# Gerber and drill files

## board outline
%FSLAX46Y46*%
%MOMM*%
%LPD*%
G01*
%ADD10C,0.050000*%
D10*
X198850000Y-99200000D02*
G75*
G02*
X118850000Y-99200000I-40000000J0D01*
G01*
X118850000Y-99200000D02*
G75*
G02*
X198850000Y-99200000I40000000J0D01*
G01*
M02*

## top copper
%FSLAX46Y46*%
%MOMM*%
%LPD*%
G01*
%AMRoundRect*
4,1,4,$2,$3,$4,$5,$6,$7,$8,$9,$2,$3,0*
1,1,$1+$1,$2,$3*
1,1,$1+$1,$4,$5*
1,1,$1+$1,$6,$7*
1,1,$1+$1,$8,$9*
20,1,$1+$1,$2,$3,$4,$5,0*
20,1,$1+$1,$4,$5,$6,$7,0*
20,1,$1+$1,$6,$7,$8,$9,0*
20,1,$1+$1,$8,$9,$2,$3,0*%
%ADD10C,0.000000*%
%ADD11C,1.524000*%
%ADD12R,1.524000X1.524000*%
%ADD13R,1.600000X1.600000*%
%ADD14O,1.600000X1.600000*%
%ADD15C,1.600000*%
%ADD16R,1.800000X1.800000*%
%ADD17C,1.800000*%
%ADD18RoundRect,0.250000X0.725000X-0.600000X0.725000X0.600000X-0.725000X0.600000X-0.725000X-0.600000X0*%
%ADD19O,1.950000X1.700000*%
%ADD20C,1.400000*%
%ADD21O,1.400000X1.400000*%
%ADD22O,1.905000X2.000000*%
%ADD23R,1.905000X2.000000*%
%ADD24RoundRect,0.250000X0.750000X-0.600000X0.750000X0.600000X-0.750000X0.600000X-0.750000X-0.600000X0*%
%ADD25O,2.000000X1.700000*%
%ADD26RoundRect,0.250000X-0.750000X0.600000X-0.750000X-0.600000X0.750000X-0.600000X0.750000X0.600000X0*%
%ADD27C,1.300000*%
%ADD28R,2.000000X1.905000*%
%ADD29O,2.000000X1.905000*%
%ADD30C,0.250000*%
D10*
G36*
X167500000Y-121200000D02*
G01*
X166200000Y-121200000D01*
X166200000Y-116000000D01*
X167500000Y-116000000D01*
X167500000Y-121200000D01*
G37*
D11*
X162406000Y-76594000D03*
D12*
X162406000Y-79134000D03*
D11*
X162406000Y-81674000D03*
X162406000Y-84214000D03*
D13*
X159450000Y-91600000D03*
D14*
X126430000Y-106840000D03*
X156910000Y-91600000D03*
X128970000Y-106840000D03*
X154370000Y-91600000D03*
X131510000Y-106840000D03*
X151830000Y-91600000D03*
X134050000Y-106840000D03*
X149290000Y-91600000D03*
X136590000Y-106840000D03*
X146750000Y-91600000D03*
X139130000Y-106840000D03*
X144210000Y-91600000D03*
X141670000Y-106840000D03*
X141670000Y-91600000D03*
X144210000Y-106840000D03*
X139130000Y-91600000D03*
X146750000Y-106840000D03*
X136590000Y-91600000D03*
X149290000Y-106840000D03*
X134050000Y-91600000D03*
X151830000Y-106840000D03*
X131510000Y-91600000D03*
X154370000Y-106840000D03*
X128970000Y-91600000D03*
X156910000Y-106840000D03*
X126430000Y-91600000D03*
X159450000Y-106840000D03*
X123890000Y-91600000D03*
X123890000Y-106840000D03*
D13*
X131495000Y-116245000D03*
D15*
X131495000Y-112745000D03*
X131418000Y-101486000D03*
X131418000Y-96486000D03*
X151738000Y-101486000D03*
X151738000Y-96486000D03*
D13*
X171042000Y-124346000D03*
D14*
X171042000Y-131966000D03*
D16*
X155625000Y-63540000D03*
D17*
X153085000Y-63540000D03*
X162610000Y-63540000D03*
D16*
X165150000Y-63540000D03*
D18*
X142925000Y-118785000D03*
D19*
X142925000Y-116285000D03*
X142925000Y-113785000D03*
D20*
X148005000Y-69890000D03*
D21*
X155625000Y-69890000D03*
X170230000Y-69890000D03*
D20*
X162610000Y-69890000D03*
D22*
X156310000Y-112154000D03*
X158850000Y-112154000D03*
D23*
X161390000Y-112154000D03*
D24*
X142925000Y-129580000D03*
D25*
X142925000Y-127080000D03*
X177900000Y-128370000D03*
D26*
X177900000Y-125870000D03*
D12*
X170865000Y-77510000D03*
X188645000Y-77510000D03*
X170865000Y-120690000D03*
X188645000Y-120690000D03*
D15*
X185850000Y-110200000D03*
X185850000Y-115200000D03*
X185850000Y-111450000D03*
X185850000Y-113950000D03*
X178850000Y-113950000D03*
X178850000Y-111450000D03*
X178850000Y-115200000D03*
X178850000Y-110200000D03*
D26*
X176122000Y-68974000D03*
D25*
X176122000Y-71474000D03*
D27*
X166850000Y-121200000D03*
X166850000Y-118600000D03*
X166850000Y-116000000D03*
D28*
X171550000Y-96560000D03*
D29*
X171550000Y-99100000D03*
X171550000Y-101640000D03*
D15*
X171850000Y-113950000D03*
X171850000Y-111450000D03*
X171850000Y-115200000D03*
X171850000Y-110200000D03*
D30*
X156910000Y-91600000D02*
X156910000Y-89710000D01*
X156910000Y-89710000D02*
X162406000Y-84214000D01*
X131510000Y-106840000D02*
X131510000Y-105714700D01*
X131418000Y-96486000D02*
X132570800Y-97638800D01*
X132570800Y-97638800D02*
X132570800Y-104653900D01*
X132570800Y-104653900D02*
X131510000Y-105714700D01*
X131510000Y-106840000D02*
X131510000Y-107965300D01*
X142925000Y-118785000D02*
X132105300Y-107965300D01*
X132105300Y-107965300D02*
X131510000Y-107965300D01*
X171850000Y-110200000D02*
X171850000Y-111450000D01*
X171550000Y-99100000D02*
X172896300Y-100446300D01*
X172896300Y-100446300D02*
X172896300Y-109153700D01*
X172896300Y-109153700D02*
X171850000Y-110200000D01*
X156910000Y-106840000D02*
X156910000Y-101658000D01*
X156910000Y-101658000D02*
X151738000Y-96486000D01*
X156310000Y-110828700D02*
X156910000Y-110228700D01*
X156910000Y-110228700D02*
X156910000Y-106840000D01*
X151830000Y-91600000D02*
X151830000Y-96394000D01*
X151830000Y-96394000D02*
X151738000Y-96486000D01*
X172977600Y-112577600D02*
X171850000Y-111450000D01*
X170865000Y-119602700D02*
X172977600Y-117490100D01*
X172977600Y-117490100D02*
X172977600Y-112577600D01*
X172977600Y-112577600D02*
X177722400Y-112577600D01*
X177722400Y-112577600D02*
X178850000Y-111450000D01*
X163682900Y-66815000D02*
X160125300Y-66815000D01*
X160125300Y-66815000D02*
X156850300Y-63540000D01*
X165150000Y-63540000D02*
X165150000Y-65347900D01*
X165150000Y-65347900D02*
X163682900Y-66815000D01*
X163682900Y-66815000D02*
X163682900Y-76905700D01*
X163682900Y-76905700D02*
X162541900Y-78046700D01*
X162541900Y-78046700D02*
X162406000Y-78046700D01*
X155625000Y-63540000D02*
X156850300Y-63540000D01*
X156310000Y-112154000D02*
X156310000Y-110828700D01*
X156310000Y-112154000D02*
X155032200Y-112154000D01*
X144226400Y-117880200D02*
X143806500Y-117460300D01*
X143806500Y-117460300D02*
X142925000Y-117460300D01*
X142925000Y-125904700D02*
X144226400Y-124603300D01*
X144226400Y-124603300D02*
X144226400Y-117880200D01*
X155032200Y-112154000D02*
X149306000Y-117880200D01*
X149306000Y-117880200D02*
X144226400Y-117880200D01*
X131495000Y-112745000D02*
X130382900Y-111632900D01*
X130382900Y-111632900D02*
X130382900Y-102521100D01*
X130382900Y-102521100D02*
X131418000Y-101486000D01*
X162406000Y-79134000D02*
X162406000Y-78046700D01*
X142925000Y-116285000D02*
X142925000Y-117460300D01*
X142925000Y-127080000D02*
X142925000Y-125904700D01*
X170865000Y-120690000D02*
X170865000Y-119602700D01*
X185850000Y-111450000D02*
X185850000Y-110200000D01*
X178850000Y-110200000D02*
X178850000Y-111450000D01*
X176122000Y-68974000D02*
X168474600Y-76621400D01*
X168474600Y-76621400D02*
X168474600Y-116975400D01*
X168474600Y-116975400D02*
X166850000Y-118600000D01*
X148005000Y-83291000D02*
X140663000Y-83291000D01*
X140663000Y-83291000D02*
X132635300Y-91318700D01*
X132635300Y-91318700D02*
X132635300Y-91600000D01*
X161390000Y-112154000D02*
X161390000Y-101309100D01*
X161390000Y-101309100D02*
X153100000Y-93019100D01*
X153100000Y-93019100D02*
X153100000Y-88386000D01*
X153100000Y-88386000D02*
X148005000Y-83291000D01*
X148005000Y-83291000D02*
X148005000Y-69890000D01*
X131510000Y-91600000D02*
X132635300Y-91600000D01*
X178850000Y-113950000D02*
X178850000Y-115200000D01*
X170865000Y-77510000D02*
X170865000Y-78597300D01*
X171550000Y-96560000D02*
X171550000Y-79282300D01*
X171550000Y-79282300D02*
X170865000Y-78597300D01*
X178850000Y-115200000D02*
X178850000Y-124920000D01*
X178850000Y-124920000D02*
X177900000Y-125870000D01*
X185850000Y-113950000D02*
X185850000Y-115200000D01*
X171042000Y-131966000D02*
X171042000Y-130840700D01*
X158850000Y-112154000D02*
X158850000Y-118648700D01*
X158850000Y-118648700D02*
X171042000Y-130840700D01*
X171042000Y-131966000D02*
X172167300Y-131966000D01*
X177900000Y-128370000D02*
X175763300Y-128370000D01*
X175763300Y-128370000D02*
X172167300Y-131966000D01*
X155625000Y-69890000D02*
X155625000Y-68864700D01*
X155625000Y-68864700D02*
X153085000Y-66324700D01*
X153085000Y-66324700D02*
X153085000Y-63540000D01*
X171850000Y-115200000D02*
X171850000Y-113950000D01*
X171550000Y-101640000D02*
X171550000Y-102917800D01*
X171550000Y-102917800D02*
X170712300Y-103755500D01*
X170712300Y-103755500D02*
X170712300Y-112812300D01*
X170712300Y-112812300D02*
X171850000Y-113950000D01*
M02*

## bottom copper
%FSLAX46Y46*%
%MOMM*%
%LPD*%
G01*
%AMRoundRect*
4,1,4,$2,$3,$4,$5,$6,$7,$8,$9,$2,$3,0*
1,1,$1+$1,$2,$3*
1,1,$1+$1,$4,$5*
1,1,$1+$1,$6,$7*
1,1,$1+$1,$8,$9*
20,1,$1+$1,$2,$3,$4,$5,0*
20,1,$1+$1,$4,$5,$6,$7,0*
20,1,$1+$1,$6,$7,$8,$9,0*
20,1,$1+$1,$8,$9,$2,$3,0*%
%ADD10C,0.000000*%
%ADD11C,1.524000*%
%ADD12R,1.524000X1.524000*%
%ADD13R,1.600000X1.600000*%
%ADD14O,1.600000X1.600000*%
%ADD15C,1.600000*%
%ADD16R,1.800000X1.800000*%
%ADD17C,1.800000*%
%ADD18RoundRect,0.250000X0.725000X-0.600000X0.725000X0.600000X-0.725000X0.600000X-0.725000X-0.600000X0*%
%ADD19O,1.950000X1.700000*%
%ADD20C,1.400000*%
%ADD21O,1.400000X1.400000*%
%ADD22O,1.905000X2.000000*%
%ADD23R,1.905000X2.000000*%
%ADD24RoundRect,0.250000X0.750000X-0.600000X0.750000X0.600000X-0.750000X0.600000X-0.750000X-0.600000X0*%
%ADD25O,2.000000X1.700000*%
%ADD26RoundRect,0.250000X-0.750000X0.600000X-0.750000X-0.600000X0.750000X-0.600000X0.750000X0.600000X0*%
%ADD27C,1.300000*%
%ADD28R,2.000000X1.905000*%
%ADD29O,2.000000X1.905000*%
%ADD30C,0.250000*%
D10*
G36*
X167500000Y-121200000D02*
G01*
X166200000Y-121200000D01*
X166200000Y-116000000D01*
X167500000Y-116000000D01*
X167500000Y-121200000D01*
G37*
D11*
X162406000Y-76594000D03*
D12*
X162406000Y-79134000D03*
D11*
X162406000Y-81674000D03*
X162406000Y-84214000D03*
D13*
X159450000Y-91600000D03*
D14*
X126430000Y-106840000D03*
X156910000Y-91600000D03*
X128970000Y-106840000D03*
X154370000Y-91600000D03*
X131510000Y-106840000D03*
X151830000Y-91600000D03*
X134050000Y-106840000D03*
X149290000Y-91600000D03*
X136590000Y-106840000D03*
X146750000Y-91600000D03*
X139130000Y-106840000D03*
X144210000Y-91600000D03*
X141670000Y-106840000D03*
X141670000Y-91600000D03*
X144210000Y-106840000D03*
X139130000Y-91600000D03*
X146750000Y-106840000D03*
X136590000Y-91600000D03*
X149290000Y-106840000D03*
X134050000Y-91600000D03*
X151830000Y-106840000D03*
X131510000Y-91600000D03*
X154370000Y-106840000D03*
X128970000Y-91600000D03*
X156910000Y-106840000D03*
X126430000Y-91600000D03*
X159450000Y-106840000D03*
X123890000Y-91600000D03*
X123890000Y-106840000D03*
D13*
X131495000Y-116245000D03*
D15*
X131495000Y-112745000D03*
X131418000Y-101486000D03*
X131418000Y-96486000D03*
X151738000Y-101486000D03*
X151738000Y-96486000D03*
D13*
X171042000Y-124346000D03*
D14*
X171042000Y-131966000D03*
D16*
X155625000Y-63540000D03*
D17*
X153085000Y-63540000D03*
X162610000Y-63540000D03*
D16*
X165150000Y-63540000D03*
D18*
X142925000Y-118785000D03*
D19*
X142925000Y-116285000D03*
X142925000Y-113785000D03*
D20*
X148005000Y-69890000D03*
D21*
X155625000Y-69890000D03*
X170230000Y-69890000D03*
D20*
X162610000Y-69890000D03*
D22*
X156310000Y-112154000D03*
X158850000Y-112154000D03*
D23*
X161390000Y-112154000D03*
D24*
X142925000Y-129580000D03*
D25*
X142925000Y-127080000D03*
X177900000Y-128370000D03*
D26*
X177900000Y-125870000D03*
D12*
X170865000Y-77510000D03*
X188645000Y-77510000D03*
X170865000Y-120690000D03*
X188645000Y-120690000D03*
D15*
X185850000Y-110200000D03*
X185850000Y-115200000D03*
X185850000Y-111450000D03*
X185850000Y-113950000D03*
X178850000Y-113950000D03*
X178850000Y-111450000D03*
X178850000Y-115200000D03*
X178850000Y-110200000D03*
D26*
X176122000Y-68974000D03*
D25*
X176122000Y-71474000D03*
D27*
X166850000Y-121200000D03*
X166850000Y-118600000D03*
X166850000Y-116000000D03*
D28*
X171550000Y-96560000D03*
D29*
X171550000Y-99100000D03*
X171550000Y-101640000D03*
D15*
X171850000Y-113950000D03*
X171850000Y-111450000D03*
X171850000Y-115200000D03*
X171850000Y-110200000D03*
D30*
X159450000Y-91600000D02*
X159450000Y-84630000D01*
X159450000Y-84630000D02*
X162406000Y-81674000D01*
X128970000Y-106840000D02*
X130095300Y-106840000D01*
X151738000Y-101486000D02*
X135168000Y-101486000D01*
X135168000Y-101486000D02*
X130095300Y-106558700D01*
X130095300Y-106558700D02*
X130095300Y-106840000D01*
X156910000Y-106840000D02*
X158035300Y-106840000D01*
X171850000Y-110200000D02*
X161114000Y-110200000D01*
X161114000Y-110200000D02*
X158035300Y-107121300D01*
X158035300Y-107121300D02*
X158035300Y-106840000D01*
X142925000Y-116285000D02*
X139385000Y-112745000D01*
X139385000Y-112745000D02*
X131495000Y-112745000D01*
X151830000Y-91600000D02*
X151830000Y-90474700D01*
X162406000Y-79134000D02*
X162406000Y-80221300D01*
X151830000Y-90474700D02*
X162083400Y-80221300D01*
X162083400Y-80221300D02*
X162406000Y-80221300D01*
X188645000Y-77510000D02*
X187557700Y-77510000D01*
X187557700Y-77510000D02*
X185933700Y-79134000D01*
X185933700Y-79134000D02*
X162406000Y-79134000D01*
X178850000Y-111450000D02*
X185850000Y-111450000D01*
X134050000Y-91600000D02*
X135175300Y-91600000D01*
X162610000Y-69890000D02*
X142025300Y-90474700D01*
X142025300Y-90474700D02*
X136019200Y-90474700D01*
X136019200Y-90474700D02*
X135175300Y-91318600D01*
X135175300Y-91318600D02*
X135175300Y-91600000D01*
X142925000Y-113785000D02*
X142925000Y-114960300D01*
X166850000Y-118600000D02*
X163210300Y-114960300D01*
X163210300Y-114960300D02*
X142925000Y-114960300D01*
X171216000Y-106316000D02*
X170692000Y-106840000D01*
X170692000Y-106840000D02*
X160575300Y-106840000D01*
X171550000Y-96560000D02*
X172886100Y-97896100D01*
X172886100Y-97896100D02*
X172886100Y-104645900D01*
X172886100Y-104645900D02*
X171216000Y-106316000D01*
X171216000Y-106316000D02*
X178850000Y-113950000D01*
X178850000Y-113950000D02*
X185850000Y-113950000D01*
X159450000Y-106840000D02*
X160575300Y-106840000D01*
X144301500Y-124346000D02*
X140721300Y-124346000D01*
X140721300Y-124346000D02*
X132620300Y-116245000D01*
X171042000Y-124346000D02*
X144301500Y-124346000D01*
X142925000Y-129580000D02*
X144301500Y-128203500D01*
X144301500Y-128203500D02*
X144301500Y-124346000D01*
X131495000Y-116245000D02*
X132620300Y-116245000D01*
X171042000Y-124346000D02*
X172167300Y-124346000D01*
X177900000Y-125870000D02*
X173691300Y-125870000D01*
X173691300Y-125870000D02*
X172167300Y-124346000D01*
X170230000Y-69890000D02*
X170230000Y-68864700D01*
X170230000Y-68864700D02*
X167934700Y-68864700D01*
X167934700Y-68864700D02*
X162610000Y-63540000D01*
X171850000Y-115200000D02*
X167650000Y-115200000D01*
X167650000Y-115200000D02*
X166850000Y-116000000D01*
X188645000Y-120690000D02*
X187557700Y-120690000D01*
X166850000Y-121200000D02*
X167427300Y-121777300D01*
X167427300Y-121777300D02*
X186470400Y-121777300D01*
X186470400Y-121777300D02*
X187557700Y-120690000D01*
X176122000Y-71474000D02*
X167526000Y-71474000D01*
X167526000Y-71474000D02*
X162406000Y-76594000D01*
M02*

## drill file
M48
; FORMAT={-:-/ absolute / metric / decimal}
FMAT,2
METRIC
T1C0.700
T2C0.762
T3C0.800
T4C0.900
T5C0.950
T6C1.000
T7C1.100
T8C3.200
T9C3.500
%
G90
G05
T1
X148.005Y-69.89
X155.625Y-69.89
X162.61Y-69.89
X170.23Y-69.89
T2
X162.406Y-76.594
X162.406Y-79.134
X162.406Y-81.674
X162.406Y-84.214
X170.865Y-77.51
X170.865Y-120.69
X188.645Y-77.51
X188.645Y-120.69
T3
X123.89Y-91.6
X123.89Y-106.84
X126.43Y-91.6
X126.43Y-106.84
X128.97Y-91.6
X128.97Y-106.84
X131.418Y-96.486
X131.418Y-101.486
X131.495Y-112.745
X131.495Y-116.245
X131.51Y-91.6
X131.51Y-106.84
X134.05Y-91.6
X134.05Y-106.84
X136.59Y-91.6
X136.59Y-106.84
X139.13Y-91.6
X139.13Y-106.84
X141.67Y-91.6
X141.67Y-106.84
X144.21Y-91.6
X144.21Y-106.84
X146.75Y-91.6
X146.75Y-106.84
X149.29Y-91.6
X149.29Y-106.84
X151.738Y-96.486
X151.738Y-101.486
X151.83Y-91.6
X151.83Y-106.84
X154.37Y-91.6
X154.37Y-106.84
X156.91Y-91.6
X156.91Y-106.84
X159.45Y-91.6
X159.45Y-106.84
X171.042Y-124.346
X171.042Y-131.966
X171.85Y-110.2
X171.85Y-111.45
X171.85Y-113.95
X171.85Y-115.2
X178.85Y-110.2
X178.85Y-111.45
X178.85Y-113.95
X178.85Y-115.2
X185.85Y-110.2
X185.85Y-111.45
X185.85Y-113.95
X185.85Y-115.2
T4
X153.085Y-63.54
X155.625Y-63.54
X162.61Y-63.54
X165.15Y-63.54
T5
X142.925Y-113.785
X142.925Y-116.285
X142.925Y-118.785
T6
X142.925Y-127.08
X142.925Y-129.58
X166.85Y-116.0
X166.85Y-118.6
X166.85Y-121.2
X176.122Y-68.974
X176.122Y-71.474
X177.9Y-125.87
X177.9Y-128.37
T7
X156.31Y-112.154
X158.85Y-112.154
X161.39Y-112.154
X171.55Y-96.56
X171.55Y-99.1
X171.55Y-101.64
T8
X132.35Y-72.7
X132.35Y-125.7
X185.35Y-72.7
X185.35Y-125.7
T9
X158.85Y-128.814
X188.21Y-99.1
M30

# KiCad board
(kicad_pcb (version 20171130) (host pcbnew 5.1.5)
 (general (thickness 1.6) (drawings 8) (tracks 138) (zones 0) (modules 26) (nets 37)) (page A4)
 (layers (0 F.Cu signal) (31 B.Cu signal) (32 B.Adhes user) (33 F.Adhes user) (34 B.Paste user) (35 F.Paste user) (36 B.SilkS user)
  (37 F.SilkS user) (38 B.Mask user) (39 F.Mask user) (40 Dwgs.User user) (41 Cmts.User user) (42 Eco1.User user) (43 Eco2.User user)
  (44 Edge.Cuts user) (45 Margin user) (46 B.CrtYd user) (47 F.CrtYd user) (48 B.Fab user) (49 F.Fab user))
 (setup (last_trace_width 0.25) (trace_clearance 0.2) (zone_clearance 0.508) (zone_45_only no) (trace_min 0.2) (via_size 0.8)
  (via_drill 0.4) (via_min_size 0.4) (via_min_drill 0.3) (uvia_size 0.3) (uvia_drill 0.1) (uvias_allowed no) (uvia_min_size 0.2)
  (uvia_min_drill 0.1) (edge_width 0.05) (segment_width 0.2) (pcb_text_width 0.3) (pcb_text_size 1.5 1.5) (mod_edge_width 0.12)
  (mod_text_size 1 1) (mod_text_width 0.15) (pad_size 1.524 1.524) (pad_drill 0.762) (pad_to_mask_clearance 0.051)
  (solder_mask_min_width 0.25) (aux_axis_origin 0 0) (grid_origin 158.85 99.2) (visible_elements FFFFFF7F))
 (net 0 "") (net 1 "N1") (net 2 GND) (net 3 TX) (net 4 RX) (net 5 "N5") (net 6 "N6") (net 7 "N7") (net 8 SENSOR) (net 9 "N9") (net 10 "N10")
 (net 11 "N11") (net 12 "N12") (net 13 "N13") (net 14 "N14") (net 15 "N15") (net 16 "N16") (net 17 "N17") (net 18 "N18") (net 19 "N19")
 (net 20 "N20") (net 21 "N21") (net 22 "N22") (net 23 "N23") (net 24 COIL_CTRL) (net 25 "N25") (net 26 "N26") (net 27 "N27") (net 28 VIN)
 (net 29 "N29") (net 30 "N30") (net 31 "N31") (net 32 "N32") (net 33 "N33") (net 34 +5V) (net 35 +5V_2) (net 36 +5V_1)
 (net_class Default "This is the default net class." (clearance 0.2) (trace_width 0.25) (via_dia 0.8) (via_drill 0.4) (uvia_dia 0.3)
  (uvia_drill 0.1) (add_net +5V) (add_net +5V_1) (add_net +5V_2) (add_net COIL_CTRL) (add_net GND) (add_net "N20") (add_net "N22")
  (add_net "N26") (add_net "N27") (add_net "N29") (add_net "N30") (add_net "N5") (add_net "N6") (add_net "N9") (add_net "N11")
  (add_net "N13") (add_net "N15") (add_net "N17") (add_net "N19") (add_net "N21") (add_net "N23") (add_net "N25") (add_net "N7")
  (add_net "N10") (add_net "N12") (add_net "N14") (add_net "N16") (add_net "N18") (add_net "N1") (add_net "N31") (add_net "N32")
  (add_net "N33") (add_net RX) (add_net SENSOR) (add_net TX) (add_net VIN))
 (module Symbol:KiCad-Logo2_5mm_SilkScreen (layer F.Cu) (at 158.85 135.2)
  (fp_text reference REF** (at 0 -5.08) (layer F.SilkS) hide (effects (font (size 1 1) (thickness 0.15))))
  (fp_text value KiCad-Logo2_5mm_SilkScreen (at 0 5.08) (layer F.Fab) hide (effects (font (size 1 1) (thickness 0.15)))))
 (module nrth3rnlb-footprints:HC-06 (layer F.Cu) (at 166.216 72.784 270)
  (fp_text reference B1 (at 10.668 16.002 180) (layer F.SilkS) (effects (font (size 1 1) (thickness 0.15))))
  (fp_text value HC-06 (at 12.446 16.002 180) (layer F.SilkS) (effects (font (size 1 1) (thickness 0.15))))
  (pad 1 thru_hole circle (at 3.81 3.81 270) (size 1.524 1.524) (drill 0.762) (layers *.Cu *.Mask) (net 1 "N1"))
  (pad 2 thru_hole rect (at 6.35 3.81 270) (size 1.524 1.524) (drill 0.762) (layers *.Cu *.Mask) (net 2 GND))
  (pad 3 thru_hole circle (at 8.89 3.81 270) (size 1.524 1.524) (drill 0.762) (layers *.Cu *.Mask) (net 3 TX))
  (pad 4 thru_hole circle (at 11.43 3.81 270) (size 1.524 1.524) (drill 0.762) (layers *.Cu *.Mask) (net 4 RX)))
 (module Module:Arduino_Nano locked (layer F.Cu) (at 159.45 91.6 270)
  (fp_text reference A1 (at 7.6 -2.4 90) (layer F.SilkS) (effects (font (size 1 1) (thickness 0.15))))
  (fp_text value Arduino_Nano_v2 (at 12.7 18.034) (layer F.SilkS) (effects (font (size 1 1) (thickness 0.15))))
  (pad 1 thru_hole rect (at 0 0 270) (size 1.6 1.6) (drill 0.8) (layers *.Cu *.Mask) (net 3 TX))
  (pad 17 thru_hole oval (at 15.24 33.02 270) (size 1.6 1.6) (drill 0.8) (layers *.Cu *.Mask) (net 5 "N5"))
  (pad 2 thru_hole oval (at 0 2.54 270) (size 1.6 1.6) (drill 0.8) (layers *.Cu *.Mask) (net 4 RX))
  (pad 18 thru_hole oval (at 15.24 30.48 270) (size 1.6 1.6) (drill 0.8) (layers *.Cu *.Mask) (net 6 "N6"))
  (pad 3 thru_hole oval (at 0 5.08 270) (size 1.6 1.6) (drill 0.8) (layers *.Cu *.Mask) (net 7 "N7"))
  (pad 19 thru_hole oval (at 15.24 27.94 270) (size 1.6 1.6) (drill 0.8) (layers *.Cu *.Mask) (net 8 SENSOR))
  (pad 4 thru_hole oval (at 0 7.62 270) (size 1.6 1.6) (drill 0.8) (layers *.Cu *.Mask) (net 2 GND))
  (pad 20 thru_hole oval (at 15.24 25.4 270) (size 1.6 1.6) (drill 0.8) (layers *.Cu *.Mask) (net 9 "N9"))
  (pad 5 thru_hole oval (at 0 10.16 270) (size 1.6 1.6) (drill 0.8) (layers *.Cu *.Mask) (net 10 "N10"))
  (pad 21 thru_hole oval (at 15.24 22.86 270) (size 1.6 1.6) (drill 0.8) (layers *.Cu *.Mask) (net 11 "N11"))
  (pad 6 thru_hole oval (at 0 12.7 270) (size 1.6 1.6) (drill 0.8) (layers *.Cu *.Mask) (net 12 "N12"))
  (pad 22 thru_hole oval (at 15.24 20.32 270) (size 1.6 1.6) (drill 0.8) (layers *.Cu *.Mask) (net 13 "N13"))
  (pad 7 thru_hole oval (at 0 15.24 270) (size 1.6 1.6) (drill 0.8) (layers *.Cu *.Mask) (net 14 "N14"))
  (pad 23 thru_hole oval (at 15.24 17.78 270) (size 1.6 1.6) (drill 0.8) (layers *.Cu *.Mask) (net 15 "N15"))
  (pad 8 thru_hole oval (at 0 17.78 270) (size 1.6 1.6) (drill 0.8) (layers *.Cu *.Mask) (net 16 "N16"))
  (pad 24 thru_hole oval (at 15.24 15.24 270) (size 1.6 1.6) (drill 0.8) (layers *.Cu *.Mask) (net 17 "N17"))
  (pad 9 thru_hole oval (at 0 20.32 270) (size 1.6 1.6) (drill 0.8) (layers *.Cu *.Mask) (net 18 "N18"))
  (pad 25 thru_hole oval (at 15.24 12.7 270) (size 1.6 1.6) (drill 0.8) (layers *.Cu *.Mask) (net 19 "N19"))
  (pad 10 thru_hole oval (at 0 22.86 270) (size 1.6 1.6) (drill 0.8) (layers *.Cu *.Mask) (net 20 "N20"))
  (pad 26 thru_hole oval (at 15.24 10.16 270) (size 1.6 1.6) (drill 0.8) (layers *.Cu *.Mask) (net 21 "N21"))
  (pad 11 thru_hole oval (at 0 25.4 270) (size 1.6 1.6) (drill 0.8) (layers *.Cu *.Mask) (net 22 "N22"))
  (pad 27 thru_hole oval (at 15.24 7.62 270) (size 1.6 1.6) (drill 0.8) (layers *.Cu *.Mask) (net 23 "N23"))
  (pad 12 thru_hole oval (at 0 27.94 270) (size 1.6 1.6) (drill 0.8) (layers *.Cu *.Mask) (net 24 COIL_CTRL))
  (pad 28 thru_hole oval (at 15.24 5.08 270) (size 1.6 1.6) (drill 0.8) (layers *.Cu *.Mask) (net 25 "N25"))
  (pad 13 thru_hole oval (at 0 30.48 270) (size 1.6 1.6) (drill 0.8) (layers *.Cu *.Mask) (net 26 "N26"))
  (pad 29 thru_hole oval (at 15.24 2.54 270) (size 1.6 1.6) (drill 0.8) (layers *.Cu *.Mask) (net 2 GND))
  (pad 14 thru_hole oval (at 0 33.02 270) (size 1.6 1.6) (drill 0.8) (layers *.Cu *.Mask) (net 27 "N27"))
  (pad 30 thru_hole oval (at 15.24 0 270) (size 1.6 1.6) (drill 0.8) (layers *.Cu *.Mask) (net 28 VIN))
  (pad 15 thru_hole oval (at 0 35.56 270) (size 1.6 1.6) (drill 0.8) (layers *.Cu *.Mask) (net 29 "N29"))
  (pad 16 thru_hole oval (at 15.24 35.56 270) (size 1.6 1.6) (drill 0.8) (layers *.Cu *.Mask) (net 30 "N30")))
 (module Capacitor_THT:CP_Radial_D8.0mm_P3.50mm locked (layer F.Cu) (at 131.495 116.245 90)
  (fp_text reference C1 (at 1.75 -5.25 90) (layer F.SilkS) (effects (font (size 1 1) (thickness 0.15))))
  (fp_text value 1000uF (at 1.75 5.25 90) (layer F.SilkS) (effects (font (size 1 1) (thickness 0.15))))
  (pad 1 thru_hole rect (at 0 0 90) (size 1.6 1.6) (drill 0.8) (layers *.Cu *.Mask) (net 28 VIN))
  (pad 2 thru_hole circle (at 3.5 0 90) (size 1.6 1.6) (drill 0.8) (layers *.Cu *.Mask) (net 2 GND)))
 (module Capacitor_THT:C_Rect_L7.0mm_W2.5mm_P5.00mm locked (layer F.Cu) (at 131.418 96.486 270)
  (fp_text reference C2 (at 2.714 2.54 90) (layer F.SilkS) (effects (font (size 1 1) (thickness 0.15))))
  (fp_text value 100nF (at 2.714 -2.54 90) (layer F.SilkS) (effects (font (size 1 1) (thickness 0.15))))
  (pad 2 thru_hole circle (at 5 0 270) (size 1.6 1.6) (drill 0.8) (layers *.Cu *.Mask) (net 2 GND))
  (pad 1 thru_hole circle (at 0 0 270) (size 1.6 1.6) (drill 0.8) (layers *.Cu *.Mask) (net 8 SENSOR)))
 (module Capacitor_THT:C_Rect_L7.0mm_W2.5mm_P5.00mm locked (layer F.Cu) (at 151.738 101.486 90)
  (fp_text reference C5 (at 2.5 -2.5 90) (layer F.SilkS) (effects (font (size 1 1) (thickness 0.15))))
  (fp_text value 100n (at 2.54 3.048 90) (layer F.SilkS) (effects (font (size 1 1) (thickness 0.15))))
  (pad 1 thru_hole circle (at 0 0 90) (size 1.6 1.6) (drill 0.8) (layers *.Cu *.Mask) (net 6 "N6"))
  (pad 2 thru_hole circle (at 5 0 90) (size 1.6 1.6) (drill 0.8) (layers *.Cu *.Mask) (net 2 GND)))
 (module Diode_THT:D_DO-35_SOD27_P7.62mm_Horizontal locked (layer F.Cu) (at 171.042 124.346 270)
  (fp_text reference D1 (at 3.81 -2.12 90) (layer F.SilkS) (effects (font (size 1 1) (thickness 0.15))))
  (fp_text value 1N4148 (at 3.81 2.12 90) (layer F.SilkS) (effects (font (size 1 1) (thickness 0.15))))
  (pad 1 thru_hole rect (at 0 0 270) (size 1.6 1.6) (drill 0.8) (layers *.Cu *.Mask) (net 28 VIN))
  (pad 2 thru_hole oval (at 7.62 0 270) (size 1.6 1.6) (drill 0.8) (layers *.Cu *.Mask) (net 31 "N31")))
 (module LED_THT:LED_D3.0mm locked (layer F.Cu) (at 155.625 63.54 180)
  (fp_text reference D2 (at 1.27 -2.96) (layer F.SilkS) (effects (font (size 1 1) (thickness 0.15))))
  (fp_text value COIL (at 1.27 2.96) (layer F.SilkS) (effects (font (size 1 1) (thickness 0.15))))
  (pad 1 thru_hole rect (at 0 0 180) (size 1.8 1.8) (drill 0.9) (layers *.Cu *.Mask) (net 2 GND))
  (pad 2 thru_hole circle (at 2.54 0 180) (size 1.8 1.8) (drill 0.9) (layers *.Cu *.Mask) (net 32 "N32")))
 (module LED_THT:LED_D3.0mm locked (layer F.Cu) (at 165.15 63.54 180)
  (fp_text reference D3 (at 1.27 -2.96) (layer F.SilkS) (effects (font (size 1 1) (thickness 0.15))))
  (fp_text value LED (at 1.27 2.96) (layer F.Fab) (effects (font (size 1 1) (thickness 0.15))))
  (pad 2 thru_hole circle (at 2.54 0 180) (size 1.8 1.8) (drill 0.9) (layers *.Cu *.Mask) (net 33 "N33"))
  (pad 1 thru_hole rect (at 0 0 180) (size 1.8 1.8) (drill 0.9) (layers *.Cu *.Mask) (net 2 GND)))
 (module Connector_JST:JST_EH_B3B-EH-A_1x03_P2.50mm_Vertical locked (layer F.Cu) (at 142.925 118.785 90)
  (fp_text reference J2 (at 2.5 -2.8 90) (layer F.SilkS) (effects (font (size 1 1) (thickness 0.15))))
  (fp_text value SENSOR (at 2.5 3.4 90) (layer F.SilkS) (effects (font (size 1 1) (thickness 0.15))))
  (pad 1 thru_hole roundrect (at 0 0 90) (size 1.7 1.95) (drill 0.95) (layers *.Cu *.Mask) (roundrect_rratio 0.147059) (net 8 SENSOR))
  (pad 2 thru_hole oval (at 2.5 0 90) (size 1.7 1.95) (drill 0.95) (layers *.Cu *.Mask) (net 2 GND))
  (pad 3 thru_hole oval (at 5 0 90) (size 1.7 1.95) (drill 0.95) (layers *.Cu *.Mask) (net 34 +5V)))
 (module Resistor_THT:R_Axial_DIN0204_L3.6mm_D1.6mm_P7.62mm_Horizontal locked (layer F.Cu) (at 148.005 69.89)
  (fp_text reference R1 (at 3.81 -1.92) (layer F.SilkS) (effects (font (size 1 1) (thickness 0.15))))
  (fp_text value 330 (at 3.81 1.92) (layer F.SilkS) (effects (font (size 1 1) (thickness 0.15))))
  (pad 1 thru_hole circle (at 0 0) (size 1.4 1.4) (drill 0.7) (layers *.Cu *.Mask) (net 24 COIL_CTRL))
  (pad 2 thru_hole oval (at 7.62 0) (size 1.4 1.4) (drill 0.7) (layers *.Cu *.Mask) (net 32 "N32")))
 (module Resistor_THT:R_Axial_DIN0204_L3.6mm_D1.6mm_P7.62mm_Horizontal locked (layer F.Cu) (at 162.61 69.89)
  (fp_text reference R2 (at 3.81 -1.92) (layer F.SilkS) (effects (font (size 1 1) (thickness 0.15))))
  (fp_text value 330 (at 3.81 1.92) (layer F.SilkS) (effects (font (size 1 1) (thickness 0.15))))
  (pad 2 thru_hole oval (at 7.62 0) (size 1.4 1.4) (drill 0.7) (layers *.Cu *.Mask) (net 33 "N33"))
  (pad 1 thru_hole circle (at 0 0) (size 1.4 1.4) (drill 0.7) (layers *.Cu *.Mask) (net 22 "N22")))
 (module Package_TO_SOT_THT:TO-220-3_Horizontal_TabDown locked (layer F.Cu) (at 161.39 112.154 180)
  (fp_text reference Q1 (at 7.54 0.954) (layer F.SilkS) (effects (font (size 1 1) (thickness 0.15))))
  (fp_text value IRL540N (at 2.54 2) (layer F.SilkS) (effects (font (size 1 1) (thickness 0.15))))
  (pad 3 thru_hole oval (at 5.08 0 180) (size 1.905 2) (drill 1.1) (layers *.Cu *.Mask) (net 2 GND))
  (pad 2 thru_hole oval (at 2.54 0 180) (size 1.905 2) (drill 1.1) (layers *.Cu *.Mask) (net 31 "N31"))
  (pad 1 thru_hole rect (at 0 0 180) (size 1.905 2) (drill 1.1) (layers *.Cu *.Mask) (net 24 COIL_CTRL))
  (pad "" np_thru_hole oval (at 2.54 -16.66 180) (size 3.5 3.5) (drill 3.5) (layers *.Cu *.Mask)))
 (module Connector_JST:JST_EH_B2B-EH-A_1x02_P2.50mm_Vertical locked (layer F.Cu) (at 142.925 129.58 90)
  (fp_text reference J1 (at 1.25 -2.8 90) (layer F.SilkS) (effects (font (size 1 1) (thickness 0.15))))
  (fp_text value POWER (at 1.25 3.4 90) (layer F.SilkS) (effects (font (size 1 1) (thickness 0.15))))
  (pad 1 thru_hole roundrect (at 0 0 90) (size 1.7 2) (drill 1) (layers *.Cu *.Mask) (roundrect_rratio 0.147059) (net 28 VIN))
  (pad 2 thru_hole oval (at 2.5 0 90) (size 1.7 2) (drill 1) (layers *.Cu *.Mask) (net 2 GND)))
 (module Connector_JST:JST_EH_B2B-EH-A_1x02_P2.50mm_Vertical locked (layer F.Cu) (at 177.9 125.87 270)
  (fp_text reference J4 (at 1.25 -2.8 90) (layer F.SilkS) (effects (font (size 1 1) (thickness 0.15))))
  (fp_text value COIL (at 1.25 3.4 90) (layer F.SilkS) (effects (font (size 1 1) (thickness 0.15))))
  (pad 2 thru_hole oval (at 2.5 0 270) (size 1.7 2) (drill 1) (layers *.Cu *.Mask) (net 31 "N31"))
  (pad 1 thru_hole roundrect (at 0 0 270) (size 1.7 2) (drill 1) (layers *.Cu *.Mask) (roundrect_rratio 0.147059) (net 28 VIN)))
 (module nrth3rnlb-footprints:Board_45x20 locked (layer F.Cu) (at 179.755 72.43)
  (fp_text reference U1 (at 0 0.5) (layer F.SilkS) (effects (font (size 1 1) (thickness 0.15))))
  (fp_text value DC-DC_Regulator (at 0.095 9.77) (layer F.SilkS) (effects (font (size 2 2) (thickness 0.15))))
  (pad 1 thru_hole rect (at -8.89 5.08) (size 1.524 1.524) (drill 0.762) (layers *.Cu *.Mask) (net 28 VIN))
  (pad 4 thru_hole rect (at 8.89 5.08) (size 1.524 1.524) (drill 0.762) (layers *.Cu *.Mask) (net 2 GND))
  (pad 2 thru_hole rect (at -8.89 48.26) (size 1.524 1.524) (drill 0.762) (layers *.Cu *.Mask) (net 2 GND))
  (pad 3 thru_hole rect (at 8.89 48.26) (size 1.524 1.524) (drill 0.762) (layers *.Cu *.Mask) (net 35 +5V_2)))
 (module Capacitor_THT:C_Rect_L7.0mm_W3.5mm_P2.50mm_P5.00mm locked (layer F.Cu) (at 185.85 115.2 90)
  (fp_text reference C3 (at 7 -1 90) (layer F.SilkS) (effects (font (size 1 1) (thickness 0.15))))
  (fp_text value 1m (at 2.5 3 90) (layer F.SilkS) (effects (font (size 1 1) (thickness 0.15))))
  (pad 2 thru_hole circle (at 5 0 90) (size 1.6 1.6) (drill 0.8) (layers *.Cu *.Mask) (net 2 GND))
  (pad 1 thru_hole circle (at 0 0 90) (size 1.6 1.6) (drill 0.8) (layers *.Cu *.Mask) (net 28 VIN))
  (pad 2 thru_hole circle (at 3.75 0 90) (size 1.6 1.6) (drill 0.8) (layers *.Cu *.Mask) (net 2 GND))
  (pad 1 thru_hole circle (at 1.25 0 90) (size 1.6 1.6) (drill 0.8) (layers *.Cu *.Mask) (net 28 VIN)))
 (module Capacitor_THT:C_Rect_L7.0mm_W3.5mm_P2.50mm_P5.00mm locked (layer F.Cu) (at 178.85 115.2 90)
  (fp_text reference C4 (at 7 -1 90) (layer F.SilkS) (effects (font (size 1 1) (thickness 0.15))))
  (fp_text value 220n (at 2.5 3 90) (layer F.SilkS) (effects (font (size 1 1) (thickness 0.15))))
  (pad 1 thru_hole circle (at 1.25 0 90) (size 1.6 1.6) (drill 0.8) (layers *.Cu *.Mask) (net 28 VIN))
  (pad 2 thru_hole circle (at 3.75 0 90) (size 1.6 1.6) (drill 0.8) (layers *.Cu *.Mask) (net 2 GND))
  (pad 1 thru_hole circle (at 0 0 90) (size 1.6 1.6) (drill 0.8) (layers *.Cu *.Mask) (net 28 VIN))
  (pad 2 thru_hole circle (at 5 0 90) (size 1.6 1.6) (drill 0.8) (layers *.Cu *.Mask) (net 2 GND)))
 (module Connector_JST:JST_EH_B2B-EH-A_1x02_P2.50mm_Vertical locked (layer F.Cu) (at 176.122 68.974 270)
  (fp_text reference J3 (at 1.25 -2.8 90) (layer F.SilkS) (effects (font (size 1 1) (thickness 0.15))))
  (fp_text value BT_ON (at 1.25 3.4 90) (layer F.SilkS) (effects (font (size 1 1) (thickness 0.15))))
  (pad 1 thru_hole roundrect (at 0 0 270) (size 1.7 2) (drill 1) (layers *.Cu *.Mask) (roundrect_rratio 0.147059) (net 34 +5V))
  (pad 2 thru_hole oval (at 2.5 0 270) (size 1.7 2) (drill 1) (layers *.Cu *.Mask) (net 1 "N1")))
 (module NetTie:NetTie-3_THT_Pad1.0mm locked (layer F.Cu) (at 166.85 121.2 90)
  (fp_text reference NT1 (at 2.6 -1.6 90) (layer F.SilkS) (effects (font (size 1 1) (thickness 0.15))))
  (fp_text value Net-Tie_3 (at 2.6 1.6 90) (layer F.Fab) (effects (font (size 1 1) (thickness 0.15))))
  (fp_poly (pts (xy 0 -0.65) (xy 5.2 -0.65) (xy 5.2 0.65) (xy 0 0.65)) (layer F.Cu) (width 0))
  (fp_poly (pts (xy 0 -0.65) (xy 5.2 -0.65) (xy 5.2 0.65) (xy 0 0.65)) (layer B.Cu) (width 0))
  (pad 1 thru_hole circle (at 0 0 90) (size 1.3 1.3) (drill 1) (layers *.Cu) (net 35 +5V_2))
  (pad 2 thru_hole circle (at 2.6 0 90) (size 1.3 1.3) (drill 1) (layers *.Cu) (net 34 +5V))
  (pad 3 thru_hole circle (at 5.2 0 90) (size 1.3 1.3) (drill 1) (layers *.Cu) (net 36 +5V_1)))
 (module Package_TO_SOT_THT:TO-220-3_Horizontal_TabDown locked (layer F.Cu) (at 171.55 96.56 270)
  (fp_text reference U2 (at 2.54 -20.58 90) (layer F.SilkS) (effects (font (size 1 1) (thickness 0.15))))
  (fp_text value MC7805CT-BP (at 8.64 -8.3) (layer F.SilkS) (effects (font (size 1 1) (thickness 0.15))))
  (pad "" np_thru_hole oval (at 2.54 -16.66 270) (size 3.5 3.5) (drill 3.5) (layers *.Cu *.Mask))
  (pad 1 thru_hole rect (at 0 0 270) (size 1.905 2) (drill 1.1) (layers *.Cu *.Mask) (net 28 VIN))
  (pad 2 thru_hole oval (at 2.54 0 270) (size 1.905 2) (drill 1.1) (layers *.Cu *.Mask) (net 2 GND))
  (pad 3 thru_hole oval (at 5.08 0 270) (size 1.905 2) (drill 1.1) (layers *.Cu *.Mask) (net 36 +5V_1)))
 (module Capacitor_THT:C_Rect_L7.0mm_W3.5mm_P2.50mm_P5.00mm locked (layer F.Cu) (at 171.85 115.2 90)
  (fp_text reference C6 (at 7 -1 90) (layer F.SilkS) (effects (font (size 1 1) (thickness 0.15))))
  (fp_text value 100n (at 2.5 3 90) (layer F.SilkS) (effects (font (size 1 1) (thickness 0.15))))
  (pad 1 thru_hole circle (at 1.25 0 90) (size 1.6 1.6) (drill 0.8) (layers *.Cu *.Mask) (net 36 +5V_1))
  (pad 2 thru_hole circle (at 3.75 0 90) (size 1.6 1.6) (drill 0.8) (layers *.Cu *.Mask) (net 2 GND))
  (pad 1 thru_hole circle (at 0 0 90) (size 1.6 1.6) (drill 0.8) (layers *.Cu *.Mask) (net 36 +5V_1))
  (pad 2 thru_hole circle (at 5 0 90) (size 1.6 1.6) (drill 0.8) (layers *.Cu *.Mask) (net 2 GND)))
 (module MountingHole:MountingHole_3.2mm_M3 (layer F.Cu) (at 185.35 125.7)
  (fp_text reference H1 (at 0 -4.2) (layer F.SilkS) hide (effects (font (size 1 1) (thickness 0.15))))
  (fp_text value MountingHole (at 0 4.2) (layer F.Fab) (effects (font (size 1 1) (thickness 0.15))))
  (pad 1 np_thru_hole circle (at 0 0) (size 3.2 3.2) (drill 3.2) (layers *.Cu *.Mask)))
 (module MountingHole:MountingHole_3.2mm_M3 (layer F.Cu) (at 132.35 72.7)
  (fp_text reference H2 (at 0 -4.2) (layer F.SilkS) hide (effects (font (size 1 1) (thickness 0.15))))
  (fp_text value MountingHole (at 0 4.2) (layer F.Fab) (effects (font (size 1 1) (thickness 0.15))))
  (pad 1 np_thru_hole circle (at 0 0) (size 3.2 3.2) (drill 3.2) (layers *.Cu *.Mask)))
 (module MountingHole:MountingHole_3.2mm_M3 (layer F.Cu) (at 132.35 125.7)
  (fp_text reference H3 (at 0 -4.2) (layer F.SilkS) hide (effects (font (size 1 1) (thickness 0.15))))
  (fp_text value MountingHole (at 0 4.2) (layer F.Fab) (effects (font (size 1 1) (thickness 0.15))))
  (pad 1 np_thru_hole circle (at 0 0) (size 3.2 3.2) (drill 3.2) (layers *.Cu *.Mask)))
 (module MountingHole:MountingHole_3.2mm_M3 (layer F.Cu) (at 185.35 72.7)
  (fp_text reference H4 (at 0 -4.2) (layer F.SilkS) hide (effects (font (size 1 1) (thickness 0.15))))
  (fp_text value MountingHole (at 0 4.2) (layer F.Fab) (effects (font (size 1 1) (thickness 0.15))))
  (pad 1 np_thru_hole circle (at 0 0) (size 3.2 3.2) (drill 3.2) (layers *.Cu *.Mask)))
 (gr_circle (center 158.85 99.2) (end 198.85 99.2) (layer Edge.Cuts) (width 0.05))
 (segment (start 159.45 91.6) (end 159.45 84.63) (width 0.25) (layer B.Cu) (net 3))
 (segment (start 159.45 84.63) (end 162.406 81.674) (width 0.25) (layer B.Cu) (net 3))
 (segment (start 156.91 91.6) (end 156.91 89.71) (width 0.25) (layer F.Cu) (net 4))
 (segment (start 156.91 89.71) (end 162.406 84.214) (width 0.25) (layer F.Cu) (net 4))
 (segment (start 128.97 106.84) (end 130.0953 106.84) (width 0.25) (layer B.Cu) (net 6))
 (segment (start 151.738 101.486) (end 135.168 101.486) (width 0.25) (layer B.Cu) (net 6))
 (segment (start 135.168 101.486) (end 130.0953 106.5587) (width 0.25) (layer B.Cu) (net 6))
 (segment (start 130.0953 106.5587) (end 130.0953 106.84) (width 0.25) (layer B.Cu) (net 6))
 (segment (start 131.51 106.84) (end 131.51 105.7147) (width 0.25) (layer F.Cu) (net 8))
 (segment (start 131.418 96.486) (end 132.5708 97.6388) (width 0.25) (layer F.Cu) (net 8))
 (segment (start 132.5708 97.6388) (end 132.5708 104.6539) (width 0.25) (layer F.Cu) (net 8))
 (segment (start 132.5708 104.6539) (end 131.51 105.7147) (width 0.25) (layer F.Cu) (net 8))
 (segment (start 131.51 106.84) (end 131.51 107.9653) (width 0.25) (layer F.Cu) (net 8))
 (segment (start 142.925 118.785) (end 132.1053 107.9653) (width 0.25) (layer F.Cu) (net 8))
 (segment (start 132.1053 107.9653) (end 131.51 107.9653) (width 0.25) (layer F.Cu) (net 8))
 (segment (start 171.85 110.2) (end 171.85 111.45) (width 0.25) (layer F.Cu) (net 2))
 (segment (start 171.55 99.1) (end 172.8963 100.4463) (width 0.25) (layer F.Cu) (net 2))
 (segment (start 172.8963 100.4463) (end 172.8963 109.1537) (width 0.25) (layer F.Cu) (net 2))
 (segment (start 172.8963 109.1537) (end 171.85 110.2) (width 0.25) (layer F.Cu) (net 2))
 (segment (start 156.91 106.84) (end 156.91 101.658) (width 0.25) (layer F.Cu) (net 2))
 (segment (start 156.91 101.658) (end 151.738 96.486) (width 0.25) (layer F.Cu) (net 2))
 (segment (start 156.31 110.8287) (end 156.91 110.2287) (width 0.25) (layer F.Cu) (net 2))
 (segment (start 156.91 110.2287) (end 156.91 106.84) (width 0.25) (layer F.Cu) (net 2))
 (segment (start 151.83 91.6) (end 151.83 96.394) (width 0.25) (layer F.Cu) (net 2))
 (segment (start 151.83 96.394) (end 151.738 96.486) (width 0.25) (layer F.Cu) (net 2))
 (segment (start 156.91 106.84) (end 158.0353 106.84) (width 0.25) (layer B.Cu) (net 2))
 (segment (start 171.85 110.2) (end 161.114 110.2) (width 0.25) (layer B.Cu) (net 2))
 (segment (start 161.114 110.2) (end 158.0353 107.1213) (width 0.25) (layer B.Cu) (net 2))
 (segment (start 158.0353 107.1213) (end 158.0353 106.84) (width 0.25) (layer B.Cu) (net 2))
 (segment (start 172.9776 112.5776) (end 171.85 111.45) (width 0.25) (layer F.Cu) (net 2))
 (segment (start 170.865 119.6027) (end 172.9776 117.4901) (width 0.25) (layer F.Cu) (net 2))
 (segment (start 172.9776 117.4901) (end 172.9776 112.5776) (width 0.25) (layer F.Cu) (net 2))
 (segment (start 172.9776 112.5776) (end 177.7224 112.5776) (width 0.25) (layer F.Cu) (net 2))
 (segment (start 177.7224 112.5776) (end 178.85 111.45) (width 0.25) (layer F.Cu) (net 2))
 (segment (start 163.6829 66.815) (end 160.1253 66.815) (width 0.25) (layer F.Cu) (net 2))
 (segment (start 160.1253 66.815) (end 156.8503 63.54) (width 0.25) (layer F.Cu) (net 2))
 (segment (start 165.15 63.54) (end 165.15 65.3479) (width 0.25) (layer F.Cu) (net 2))
 (segment (start 165.15 65.3479) (end 163.6829 66.815) (width 0.25) (layer F.Cu) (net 2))
 (segment (start 163.6829 66.815) (end 163.6829 76.9057) (width 0.25) (layer F.Cu) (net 2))
 (segment (start 163.6829 76.9057) (end 162.5419 78.0467) (width 0.25) (layer F.Cu) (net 2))
 (segment (start 162.5419 78.0467) (end 162.406 78.0467) (width 0.25) (layer F.Cu) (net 2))
 (segment (start 155.625 63.54) (end 156.8503 63.54) (width 0.25) (layer F.Cu) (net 2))
 (segment (start 156.31 112.154) (end 156.31 110.8287) (width 0.25) (layer F.Cu) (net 2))
 (segment (start 142.925 116.285) (end 139.385 112.745) (width 0.25) (layer B.Cu) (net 2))
 (segment (start 139.385 112.745) (end 131.495 112.745) (width 0.25) (layer B.Cu) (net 2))
 (segment (start 156.31 112.154) (end 155.0322 112.154) (width 0.25) (layer F.Cu) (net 2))
 (segment (start 144.2264 117.8802) (end 143.8065 117.4603) (width 0.25) (layer F.Cu) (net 2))
 (segment (start 143.8065 117.4603) (end 142.925 117.4603) (width 0.25) (layer F.Cu) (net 2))
 (segment (start 142.925 125.9047) (end 144.2264 124.6033) (width 0.25) (layer F.Cu) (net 2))
 (segment (start 144.2264 124.6033) (end 144.2264 117.8802) (width 0.25) (layer F.Cu) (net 2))
 (segment (start 155.0322 112.154) (end 149.306 117.8802) (width 0.25) (layer F.Cu) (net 2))
 (segment (start 149.306 117.8802) (end 144.2264 117.8802) (width 0.25) (layer F.Cu) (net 2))
 (segment (start 131.495 112.745) (end 130.3829 111.6329) (width 0.25) (layer F.Cu) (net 2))
 (segment (start 130.3829 111.6329) (end 130.3829 102.5211) (width 0.25) (layer F.Cu) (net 2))
 (segment (start 130.3829 102.5211) (end 131.418 101.486) (width 0.25) (layer F.Cu) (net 2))
 (segment (start 151.83 91.6) (end 151.83 90.4747) (width 0.25) (layer B.Cu) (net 2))
 (segment (start 162.406 79.134) (end 162.406 80.2213) (width 0.25) (layer B.Cu) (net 2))
 (segment (start 151.83 90.4747) (end 162.0834 80.2213) (width 0.25) (layer B.Cu) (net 2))
 (segment (start 162.0834 80.2213) (end 162.406 80.2213) (width 0.25) (layer B.Cu) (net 2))
 (segment (start 162.406 79.134) (end 162.406 78.0467) (width 0.25) (layer F.Cu) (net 2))
 (segment (start 142.925 116.285) (end 142.925 117.4603) (width 0.25) (layer F.Cu) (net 2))
 (segment (start 142.925 127.08) (end 142.925 125.9047) (width 0.25) (layer F.Cu) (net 2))
 (segment (start 188.645 77.51) (end 187.5577 77.51) (width 0.25) (layer B.Cu) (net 2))
 (segment (start 187.5577 77.51) (end 185.9337 79.134) (width 0.25) (layer B.Cu) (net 2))
 (segment (start 185.9337 79.134) (end 162.406 79.134) (width 0.25) (layer B.Cu) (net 2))
 (segment (start 170.865 120.69) (end 170.865 119.6027) (width 0.25) (layer F.Cu) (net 2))
 (segment (start 185.85 111.45) (end 185.85 110.2) (width 0.25) (layer F.Cu) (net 2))
 (segment (start 178.85 111.45) (end 185.85 111.45) (width 0.25) (layer B.Cu) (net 2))
 (segment (start 178.85 110.2) (end 178.85 111.45) (width 0.25) (layer F.Cu) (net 2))
 (segment (start 134.05 91.6) (end 135.1753 91.6) (width 0.25) (layer B.Cu) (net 22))
 (segment (start 162.61 69.89) (end 142.0253 90.4747) (width 0.25) (layer B.Cu) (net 22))
 (segment (start 142.0253 90.4747) (end 136.0192 90.4747) (width 0.25) (layer B.Cu) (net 22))
 (segment (start 136.0192 90.4747) (end 135.1753 91.3186) (width 0.25) (layer B.Cu) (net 22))
 (segment (start 135.1753 91.3186) (end 135.1753 91.6) (width 0.25) (layer B.Cu) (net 22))
 (segment (start 142.925 113.785) (end 142.925 114.9603) (width 0.25) (layer B.Cu) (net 34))
 (segment (start 166.85 118.6) (end 163.2103 114.9603) (width 0.25) (layer B.Cu) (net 34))
 (segment (start 163.2103 114.9603) (end 142.925 114.9603) (width 0.25) (layer B.Cu) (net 34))
 (segment (start 176.122 68.974) (end 168.4746 76.6214) (width 0.25) (layer F.Cu) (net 34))
 (segment (start 168.4746 76.6214) (end 168.4746 116.9754) (width 0.25) (layer F.Cu) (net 34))
 (segment (start 168.4746 116.9754) (end 166.85 118.6) (width 0.25) (layer F.Cu) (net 34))
 (segment (start 148.005 83.291) (end 140.663 83.291) (width 0.25) (layer F.Cu) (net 24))
 (segment (start 140.663 83.291) (end 132.6353 91.3187) (width 0.25) (layer F.Cu) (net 24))
 (segment (start 132.6353 91.3187) (end 132.6353 91.6) (width 0.25) (layer F.Cu) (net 24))
 (segment (start 161.39 112.154) (end 161.39 101.3091) (width 0.25) (layer F.Cu) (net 24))
 (segment (start 161.39 101.3091) (end 153.1 93.0191) (width 0.25) (layer F.Cu) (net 24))
 (segment (start 153.1 93.0191) (end 153.1 88.386) (width 0.25) (layer F.Cu) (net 24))
 (segment (start 153.1 88.386) (end 148.005 83.291) (width 0.25) (layer F.Cu) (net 24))
 (segment (start 148.005 83.291) (end 148.005 69.89) (width 0.25) (layer F.Cu) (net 24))
 (segment (start 131.51 91.6) (end 132.6353 91.6) (width 0.25) (layer F.Cu) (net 24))
 (segment (start 171.216 106.316) (end 170.692 106.84) (width 0.25) (layer B.Cu) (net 28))
 (segment (start 170.692 106.84) (end 160.5753 106.84) (width 0.25) (layer B.Cu) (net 28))
 (segment (start 171.55 96.56) (end 172.8861 97.8961) (width 0.25) (layer B.Cu) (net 28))
 (segment (start 172.8861 97.8961) (end 172.8861 104.6459) (width 0.25) (layer B.Cu) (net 28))
 (segment (start 172.8861 104.6459) (end 171.216 106.316) (width 0.25) (layer B.Cu) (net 28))
 (segment (start 171.216 106.316) (end 178.85 113.95) (width 0.25) (layer B.Cu) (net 28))
 (segment (start 178.85 113.95) (end 185.85 113.95) (width 0.25) (layer B.Cu) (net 28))
 (segment (start 159.45 106.84) (end 160.5753 106.84) (width 0.25) (layer B.Cu) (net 28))
 (segment (start 178.85 113.95) (end 178.85 115.2) (width 0.25) (layer F.Cu) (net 28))
 (segment (start 170.865 77.51) (end 170.865 78.5973) (width 0.25) (layer F.Cu) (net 28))
 (segment (start 171.55 96.56) (end 171.55 79.2823) (width 0.25) (layer F.Cu) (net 28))
 (segment (start 171.55 79.2823) (end 170.865 78.5973) (width 0.25) (layer F.Cu) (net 28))
 (segment (start 144.3015 124.346) (end 140.7213 124.346) (width 0.25) (layer B.Cu) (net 28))
 (segment (start 140.7213 124.346) (end 132.6203 116.245) (width 0.25) (layer B.Cu) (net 28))
 (segment (start 171.042 124.346) (end 144.3015 124.346) (width 0.25) (layer B.Cu) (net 28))
 (segment (start 142.925 129.58) (end 144.3015 128.2035) (width 0.25) (layer B.Cu) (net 28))
 (segment (start 144.3015 128.2035) (end 144.3015 124.346) (width 0.25) (layer B.Cu) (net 28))
 (segment (start 131.495 116.245) (end 132.6203 116.245) (width 0.25) (layer B.Cu) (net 28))
 (segment (start 171.042 124.346) (end 172.1673 124.346) (width 0.25) (layer B.Cu) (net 28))
 (segment (start 177.9 125.87) (end 173.6913 125.87) (width 0.25) (layer B.Cu) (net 28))
 (segment (start 173.6913 125.87) (end 172.1673 124.346) (width 0.25) (layer B.Cu) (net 28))
 (segment (start 178.85 115.2) (end 178.85 124.92) (width 0.25) (layer F.Cu) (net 28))
 (segment (start 178.85 124.92) (end 177.9 125.87) (width 0.25) (layer F.Cu) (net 28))
 (segment (start 185.85 113.95) (end 185.85 115.2) (width 0.25) (layer F.Cu) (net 28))
 (segment (start 171.042 131.966) (end 171.042 130.8407) (width 0.25) (layer F.Cu) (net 31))
 (segment (start 158.85 112.154) (end 158.85 118.6487) (width 0.25) (layer F.Cu) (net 31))
 (segment (start 158.85 118.6487) (end 171.042 130.8407) (width 0.25) (layer F.Cu) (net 31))
 (segment (start 171.042 131.966) (end 172.1673 131.966) (width 0.25) (layer F.Cu) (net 31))
 (segment (start 177.9 128.37) (end 175.7633 128.37) (width 0.25) (layer F.Cu) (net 31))
 (segment (start 175.7633 128.37) (end 172.1673 131.966) (width 0.25) (layer F.Cu) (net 31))
 (segment (start 155.625 69.89) (end 155.625 68.8647) (width 0.25) (layer F.Cu) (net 32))
 (segment (start 155.625 68.8647) (end 153.085 66.3247) (width 0.25) (layer F.Cu) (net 32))
 (segment (start 153.085 66.3247) (end 153.085 63.54) (width 0.25) (layer F.Cu) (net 32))
 (segment (start 170.23 69.89) (end 170.23 68.8647) (width 0.25) (layer B.Cu) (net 33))
 (segment (start 170.23 68.8647) (end 167.9347 68.8647) (width 0.25) (layer B.Cu) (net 33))
 (segment (start 167.9347 68.8647) (end 162.61 63.54) (width 0.25) (layer B.Cu) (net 33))
 (segment (start 171.85 115.2) (end 167.65 115.2) (width 0.25) (layer B.Cu) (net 36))
 (segment (start 167.65 115.2) (end 166.85 116) (width 0.25) (layer B.Cu) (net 36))
 (segment (start 171.85 115.2) (end 171.85 113.95) (width 0.25) (layer F.Cu) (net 36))
 (segment (start 171.55 101.64) (end 171.55 102.9178) (width 0.25) (layer F.Cu) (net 36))
 (segment (start 171.55 102.9178) (end 170.7123 103.7555) (width 0.25) (layer F.Cu) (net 36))
 (segment (start 170.7123 103.7555) (end 170.7123 112.8123) (width 0.25) (layer F.Cu) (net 36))
 (segment (start 170.7123 112.8123) (end 171.85 113.95) (width 0.25) (layer F.Cu) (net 36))
 (segment (start 188.645 120.69) (end 187.5577 120.69) (width 0.25) (layer B.Cu) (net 35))
 (segment (start 166.85 121.2) (end 167.4273 121.7773) (width 0.25) (layer B.Cu) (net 35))
 (segment (start 167.4273 121.7773) (end 186.4704 121.7773) (width 0.25) (layer B.Cu) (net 35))
 (segment (start 186.4704 121.7773) (end 187.5577 120.69) (width 0.25) (layer B.Cu) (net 35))
 (segment (start 176.122 71.474) (end 167.526 71.474) (width 0.25) (layer B.Cu) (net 1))
 (segment (start 167.526 71.474) (end 162.406 76.594) (width 0.25) (layer B.Cu) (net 1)))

